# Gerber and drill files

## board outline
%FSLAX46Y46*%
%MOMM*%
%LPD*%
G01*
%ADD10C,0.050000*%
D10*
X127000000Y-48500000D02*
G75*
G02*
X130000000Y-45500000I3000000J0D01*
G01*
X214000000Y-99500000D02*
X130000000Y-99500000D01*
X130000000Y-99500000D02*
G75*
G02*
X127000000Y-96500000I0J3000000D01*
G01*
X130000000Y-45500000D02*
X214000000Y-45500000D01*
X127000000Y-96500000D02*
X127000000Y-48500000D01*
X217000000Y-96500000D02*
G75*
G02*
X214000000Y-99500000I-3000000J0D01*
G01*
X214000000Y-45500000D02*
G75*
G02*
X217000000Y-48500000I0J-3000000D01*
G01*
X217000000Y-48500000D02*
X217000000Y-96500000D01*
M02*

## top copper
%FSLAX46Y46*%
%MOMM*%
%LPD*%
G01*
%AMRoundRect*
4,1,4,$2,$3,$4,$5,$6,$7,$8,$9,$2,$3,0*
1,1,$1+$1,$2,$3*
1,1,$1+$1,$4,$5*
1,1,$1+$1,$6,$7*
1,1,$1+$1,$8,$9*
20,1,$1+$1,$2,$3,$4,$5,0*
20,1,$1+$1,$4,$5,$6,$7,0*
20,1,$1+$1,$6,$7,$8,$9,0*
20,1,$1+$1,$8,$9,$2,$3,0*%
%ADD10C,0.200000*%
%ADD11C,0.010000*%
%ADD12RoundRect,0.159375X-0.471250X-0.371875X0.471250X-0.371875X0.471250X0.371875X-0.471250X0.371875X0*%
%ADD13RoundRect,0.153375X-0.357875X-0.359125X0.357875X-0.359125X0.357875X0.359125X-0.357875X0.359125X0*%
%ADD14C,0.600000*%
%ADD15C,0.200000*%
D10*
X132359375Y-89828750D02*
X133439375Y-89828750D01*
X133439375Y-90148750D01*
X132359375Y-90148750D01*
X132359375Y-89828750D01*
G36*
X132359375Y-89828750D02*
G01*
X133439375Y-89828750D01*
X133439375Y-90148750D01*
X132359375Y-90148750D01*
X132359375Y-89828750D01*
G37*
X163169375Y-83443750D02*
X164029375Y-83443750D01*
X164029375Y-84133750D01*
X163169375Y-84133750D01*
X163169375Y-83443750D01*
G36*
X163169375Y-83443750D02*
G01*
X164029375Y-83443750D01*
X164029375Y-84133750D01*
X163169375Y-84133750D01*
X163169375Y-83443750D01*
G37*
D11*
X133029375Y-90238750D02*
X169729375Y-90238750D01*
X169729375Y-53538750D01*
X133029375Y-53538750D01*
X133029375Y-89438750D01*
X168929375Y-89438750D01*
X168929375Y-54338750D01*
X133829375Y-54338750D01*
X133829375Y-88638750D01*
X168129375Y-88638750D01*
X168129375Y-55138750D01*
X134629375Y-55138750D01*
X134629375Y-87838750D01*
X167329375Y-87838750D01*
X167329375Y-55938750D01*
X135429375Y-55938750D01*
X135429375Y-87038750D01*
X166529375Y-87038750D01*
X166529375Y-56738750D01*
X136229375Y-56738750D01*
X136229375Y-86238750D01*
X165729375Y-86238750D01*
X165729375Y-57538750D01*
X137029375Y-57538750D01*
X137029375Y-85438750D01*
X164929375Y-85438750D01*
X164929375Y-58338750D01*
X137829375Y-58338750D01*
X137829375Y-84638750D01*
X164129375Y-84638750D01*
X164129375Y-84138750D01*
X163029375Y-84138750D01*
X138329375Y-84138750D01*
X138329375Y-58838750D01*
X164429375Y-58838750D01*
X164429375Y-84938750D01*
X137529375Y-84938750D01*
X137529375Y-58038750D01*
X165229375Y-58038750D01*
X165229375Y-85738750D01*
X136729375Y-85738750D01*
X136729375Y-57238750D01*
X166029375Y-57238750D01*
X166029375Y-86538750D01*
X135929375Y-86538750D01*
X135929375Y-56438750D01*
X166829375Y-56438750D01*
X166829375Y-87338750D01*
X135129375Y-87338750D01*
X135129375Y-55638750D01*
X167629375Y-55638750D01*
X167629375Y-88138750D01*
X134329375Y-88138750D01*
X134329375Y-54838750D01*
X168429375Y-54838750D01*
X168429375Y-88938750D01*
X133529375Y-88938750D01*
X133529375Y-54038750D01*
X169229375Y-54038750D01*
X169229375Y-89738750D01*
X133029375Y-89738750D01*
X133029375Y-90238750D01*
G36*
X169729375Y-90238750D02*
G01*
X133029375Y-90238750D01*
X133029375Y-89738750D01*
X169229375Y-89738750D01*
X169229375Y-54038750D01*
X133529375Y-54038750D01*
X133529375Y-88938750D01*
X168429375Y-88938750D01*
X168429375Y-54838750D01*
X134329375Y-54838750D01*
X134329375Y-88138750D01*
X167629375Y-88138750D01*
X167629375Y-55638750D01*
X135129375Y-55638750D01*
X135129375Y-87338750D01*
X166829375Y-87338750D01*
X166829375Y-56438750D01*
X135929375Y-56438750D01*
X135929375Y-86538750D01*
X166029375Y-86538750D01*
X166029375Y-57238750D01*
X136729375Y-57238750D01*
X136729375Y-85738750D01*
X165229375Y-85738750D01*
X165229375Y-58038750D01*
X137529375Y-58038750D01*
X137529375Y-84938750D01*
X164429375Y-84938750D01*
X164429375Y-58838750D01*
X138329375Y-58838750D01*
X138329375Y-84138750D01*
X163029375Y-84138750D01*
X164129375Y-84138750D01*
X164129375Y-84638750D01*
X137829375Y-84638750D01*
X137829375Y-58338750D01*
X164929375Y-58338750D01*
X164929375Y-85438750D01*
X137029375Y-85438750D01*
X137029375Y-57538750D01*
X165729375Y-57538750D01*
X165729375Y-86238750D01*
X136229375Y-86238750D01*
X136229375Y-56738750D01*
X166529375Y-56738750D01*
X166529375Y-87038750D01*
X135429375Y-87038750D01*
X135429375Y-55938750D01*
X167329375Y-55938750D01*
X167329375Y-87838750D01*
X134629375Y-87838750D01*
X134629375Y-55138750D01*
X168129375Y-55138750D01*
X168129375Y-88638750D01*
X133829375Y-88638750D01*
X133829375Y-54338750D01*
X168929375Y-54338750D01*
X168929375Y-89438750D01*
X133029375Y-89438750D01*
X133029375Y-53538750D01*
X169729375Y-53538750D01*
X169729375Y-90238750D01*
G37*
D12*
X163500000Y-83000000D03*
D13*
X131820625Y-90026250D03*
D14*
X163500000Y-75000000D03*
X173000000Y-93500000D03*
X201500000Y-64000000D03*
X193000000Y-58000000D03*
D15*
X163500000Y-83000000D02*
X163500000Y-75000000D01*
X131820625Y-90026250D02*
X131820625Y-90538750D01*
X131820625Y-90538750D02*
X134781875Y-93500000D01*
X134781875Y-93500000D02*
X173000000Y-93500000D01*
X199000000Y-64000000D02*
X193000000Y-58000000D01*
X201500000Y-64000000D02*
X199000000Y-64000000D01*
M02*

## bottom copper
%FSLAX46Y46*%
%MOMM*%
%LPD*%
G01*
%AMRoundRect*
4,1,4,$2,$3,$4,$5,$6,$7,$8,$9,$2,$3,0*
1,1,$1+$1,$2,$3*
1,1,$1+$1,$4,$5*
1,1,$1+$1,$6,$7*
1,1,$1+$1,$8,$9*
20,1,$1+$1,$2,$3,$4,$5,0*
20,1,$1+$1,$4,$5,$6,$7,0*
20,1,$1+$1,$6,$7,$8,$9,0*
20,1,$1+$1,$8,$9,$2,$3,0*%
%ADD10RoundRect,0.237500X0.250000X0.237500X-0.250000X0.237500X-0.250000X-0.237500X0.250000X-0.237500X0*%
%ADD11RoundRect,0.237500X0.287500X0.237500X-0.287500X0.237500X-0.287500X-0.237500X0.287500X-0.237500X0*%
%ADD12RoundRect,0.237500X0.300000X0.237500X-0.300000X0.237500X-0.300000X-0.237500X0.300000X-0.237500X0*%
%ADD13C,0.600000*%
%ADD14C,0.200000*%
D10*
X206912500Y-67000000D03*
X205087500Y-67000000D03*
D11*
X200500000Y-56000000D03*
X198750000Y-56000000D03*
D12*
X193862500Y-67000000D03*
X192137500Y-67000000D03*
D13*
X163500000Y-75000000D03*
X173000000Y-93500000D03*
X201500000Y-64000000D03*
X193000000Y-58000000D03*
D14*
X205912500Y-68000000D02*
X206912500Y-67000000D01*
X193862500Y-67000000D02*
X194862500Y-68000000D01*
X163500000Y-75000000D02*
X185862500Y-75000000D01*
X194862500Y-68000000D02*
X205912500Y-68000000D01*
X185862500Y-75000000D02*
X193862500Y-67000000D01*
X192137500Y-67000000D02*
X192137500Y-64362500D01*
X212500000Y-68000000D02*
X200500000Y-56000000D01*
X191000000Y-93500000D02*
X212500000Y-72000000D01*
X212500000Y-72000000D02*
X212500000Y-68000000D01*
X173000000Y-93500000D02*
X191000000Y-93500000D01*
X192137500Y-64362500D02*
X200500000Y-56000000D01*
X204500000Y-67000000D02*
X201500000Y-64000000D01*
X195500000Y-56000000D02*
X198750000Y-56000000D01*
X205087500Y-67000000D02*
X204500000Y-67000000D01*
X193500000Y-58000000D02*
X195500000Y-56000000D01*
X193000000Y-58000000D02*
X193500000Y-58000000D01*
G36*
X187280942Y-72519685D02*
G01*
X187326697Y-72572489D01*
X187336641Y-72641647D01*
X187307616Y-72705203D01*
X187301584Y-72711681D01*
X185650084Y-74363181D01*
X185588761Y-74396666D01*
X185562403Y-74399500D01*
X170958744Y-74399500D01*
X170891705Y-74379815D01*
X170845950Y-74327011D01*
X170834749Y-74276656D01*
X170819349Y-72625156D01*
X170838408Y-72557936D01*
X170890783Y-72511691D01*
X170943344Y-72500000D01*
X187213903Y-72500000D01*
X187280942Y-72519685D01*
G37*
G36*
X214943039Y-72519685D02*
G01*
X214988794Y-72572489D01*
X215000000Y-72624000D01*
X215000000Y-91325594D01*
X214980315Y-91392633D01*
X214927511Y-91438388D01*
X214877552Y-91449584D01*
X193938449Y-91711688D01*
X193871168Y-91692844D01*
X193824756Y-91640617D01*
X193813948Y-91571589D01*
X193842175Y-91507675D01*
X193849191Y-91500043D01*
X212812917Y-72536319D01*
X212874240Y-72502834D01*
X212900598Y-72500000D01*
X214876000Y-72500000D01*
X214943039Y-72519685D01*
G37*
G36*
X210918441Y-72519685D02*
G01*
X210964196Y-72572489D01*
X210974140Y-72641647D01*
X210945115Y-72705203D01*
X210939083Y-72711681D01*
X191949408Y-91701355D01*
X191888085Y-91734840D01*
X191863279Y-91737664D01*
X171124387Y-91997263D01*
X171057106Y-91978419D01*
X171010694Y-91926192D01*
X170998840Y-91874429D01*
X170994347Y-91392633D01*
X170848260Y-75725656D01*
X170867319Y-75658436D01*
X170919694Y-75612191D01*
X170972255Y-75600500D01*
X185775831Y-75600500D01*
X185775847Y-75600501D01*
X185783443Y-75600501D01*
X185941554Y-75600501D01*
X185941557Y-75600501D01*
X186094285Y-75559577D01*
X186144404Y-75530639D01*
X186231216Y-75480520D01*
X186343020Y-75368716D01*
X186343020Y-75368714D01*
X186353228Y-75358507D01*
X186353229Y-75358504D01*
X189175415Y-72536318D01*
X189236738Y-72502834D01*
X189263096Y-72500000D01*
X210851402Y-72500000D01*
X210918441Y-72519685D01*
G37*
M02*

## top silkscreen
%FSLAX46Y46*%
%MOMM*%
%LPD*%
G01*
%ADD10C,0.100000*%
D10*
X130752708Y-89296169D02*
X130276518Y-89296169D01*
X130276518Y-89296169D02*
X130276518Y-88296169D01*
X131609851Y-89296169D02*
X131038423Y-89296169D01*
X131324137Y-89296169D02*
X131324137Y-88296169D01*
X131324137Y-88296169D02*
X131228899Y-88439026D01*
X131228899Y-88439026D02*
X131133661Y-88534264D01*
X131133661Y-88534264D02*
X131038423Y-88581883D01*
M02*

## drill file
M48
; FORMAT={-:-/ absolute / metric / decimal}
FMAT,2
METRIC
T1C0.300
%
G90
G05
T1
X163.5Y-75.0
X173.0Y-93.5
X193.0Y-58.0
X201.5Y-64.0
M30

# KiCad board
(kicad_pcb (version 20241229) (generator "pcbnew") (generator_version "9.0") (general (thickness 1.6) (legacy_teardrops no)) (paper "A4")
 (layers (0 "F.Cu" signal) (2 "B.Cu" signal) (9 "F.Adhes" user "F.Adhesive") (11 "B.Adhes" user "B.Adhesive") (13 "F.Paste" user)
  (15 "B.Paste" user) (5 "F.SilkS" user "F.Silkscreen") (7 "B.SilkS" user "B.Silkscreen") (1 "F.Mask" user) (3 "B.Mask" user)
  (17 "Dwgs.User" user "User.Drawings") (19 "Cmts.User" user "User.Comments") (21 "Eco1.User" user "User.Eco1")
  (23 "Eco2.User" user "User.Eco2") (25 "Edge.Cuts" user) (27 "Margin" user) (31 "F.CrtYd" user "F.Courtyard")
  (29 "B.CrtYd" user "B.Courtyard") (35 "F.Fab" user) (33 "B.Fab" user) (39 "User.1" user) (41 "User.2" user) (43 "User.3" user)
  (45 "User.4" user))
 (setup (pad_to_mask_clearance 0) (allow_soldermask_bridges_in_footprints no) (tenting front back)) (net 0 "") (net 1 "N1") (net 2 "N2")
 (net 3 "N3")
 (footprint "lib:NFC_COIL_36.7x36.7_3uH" (layer "F.Cu") (at 133.029375 90.23875)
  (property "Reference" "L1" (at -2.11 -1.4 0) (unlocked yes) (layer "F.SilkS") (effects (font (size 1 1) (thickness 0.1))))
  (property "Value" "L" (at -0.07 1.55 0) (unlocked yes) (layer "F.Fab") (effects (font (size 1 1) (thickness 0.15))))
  (fp_rect (start -0.67 -0.41) (end 0.41 -0.09) (stroke (width 0.2) (type solid)) (fill yes) (layer "F.Cu"))
  (fp_rect (start 30.14 -6.795) (end 31 -6.105) (stroke (width 0.2) (type solid)) (fill yes) (layer "F.Cu"))
  (fp_poly
   (pts (xy 0 0) (xy 36.7 0) (xy 36.7 -36.7) (xy 0 -36.7) (xy 0 -0.8) (xy 35.9 -0.8) (xy 35.9 -35.9) (xy 0.8 -35.9) (xy 0.8 -1.6)
    (xy 35.1 -1.6) (xy 35.1 -35.1) (xy 1.6 -35.1) (xy 1.6 -2.4) (xy 34.3 -2.4) (xy 34.3 -34.3) (xy 2.4 -34.3) (xy 2.4 -3.2) (xy 33.5 -3.2)
    (xy 33.5 -33.5) (xy 3.2 -33.5) (xy 3.2 -4) (xy 32.7 -4) (xy 32.7 -32.7) (xy 4 -32.7) (xy 4 -4.8) (xy 31.9 -4.8) (xy 31.9 -31.9)
    (xy 4.8 -31.9) (xy 4.8 -5.6) (xy 31.1 -5.6) (xy 31.1 -6.1) (xy 30 -6.1) (xy 5.3 -6.1) (xy 5.3 -31.4) (xy 31.4 -31.4) (xy 31.4 -5.3)
    (xy 4.5 -5.3) (xy 4.5 -32.2) (xy 32.2 -32.2) (xy 32.2 -4.5) (xy 3.7 -4.5) (xy 3.7 -33) (xy 33 -33) (xy 33 -3.7) (xy 2.9 -3.7)
    (xy 2.9 -33.8) (xy 33.8 -33.8) (xy 33.8 -2.9) (xy 2.1 -2.9) (xy 2.1 -34.6) (xy 34.6 -34.6) (xy 34.6 -2.1) (xy 1.3 -2.1) (xy 1.3 -35.4)
    (xy 35.4 -35.4) (xy 35.4 -1.3) (xy 0.5 -1.3) (xy 0.5 -36.2) (xy 36.2 -36.2) (xy 36.2 -0.5) (xy 0 -0.5))
   (stroke (width 0.01) (type solid)) (fill yes) (layer "F.Cu"))
  (pad "1" smd roundrect (at 30.470625 -7.23875) (size 1.26125 1.0625) (layers "F.Cu" "F.Mask" "F.Paste") (roundrect_rratio 0.15)
   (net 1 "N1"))
  (pad "2" smd roundrect (at -1.20875 -0.2125) (size 1.0225 1.025) (layers "F.Cu" "F.Mask" "F.Paste") (roundrect_rratio 0.15) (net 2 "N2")))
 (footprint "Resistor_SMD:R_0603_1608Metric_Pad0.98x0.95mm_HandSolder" (layer "B.Cu") (at 206 67 180)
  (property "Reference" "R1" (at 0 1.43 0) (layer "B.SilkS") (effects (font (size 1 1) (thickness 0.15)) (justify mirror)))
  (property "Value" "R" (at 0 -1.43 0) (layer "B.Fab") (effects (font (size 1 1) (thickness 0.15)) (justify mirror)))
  (pad "1" smd roundrect (at -0.9125 0 180) (size 0.975 0.95) (layers "B.Cu" "B.Mask" "B.Paste") (roundrect_rratio 0.25) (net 1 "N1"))
  (pad "2" smd roundrect (at 0.9125 0 180) (size 0.975 0.95) (layers "B.Cu" "B.Mask" "B.Paste") (roundrect_rratio 0.25) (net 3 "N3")))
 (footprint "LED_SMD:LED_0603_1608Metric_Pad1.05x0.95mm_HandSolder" (layer "B.Cu") (at 199.625 56 180)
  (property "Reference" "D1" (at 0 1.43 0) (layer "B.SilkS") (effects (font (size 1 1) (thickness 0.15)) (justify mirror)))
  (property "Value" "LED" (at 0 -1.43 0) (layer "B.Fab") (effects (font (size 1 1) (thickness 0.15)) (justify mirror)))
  (pad "1" smd roundrect (at -0.875 0 180) (size 1.05 0.95) (layers "B.Cu" "B.Mask" "B.Paste") (roundrect_rratio 0.25) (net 2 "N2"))
  (pad "2" smd roundrect (at 0.875 0 180) (size 1.05 0.95) (layers "B.Cu" "B.Mask" "B.Paste") (roundrect_rratio 0.25) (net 3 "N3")))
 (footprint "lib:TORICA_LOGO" (layer "B.Cu") (at 193 59.5 180)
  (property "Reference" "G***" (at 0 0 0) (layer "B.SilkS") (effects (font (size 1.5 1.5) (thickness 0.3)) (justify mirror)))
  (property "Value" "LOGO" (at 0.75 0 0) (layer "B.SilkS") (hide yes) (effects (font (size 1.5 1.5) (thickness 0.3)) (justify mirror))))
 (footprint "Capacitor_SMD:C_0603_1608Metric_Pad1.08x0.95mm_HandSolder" (layer "B.Cu") (at 193 67 180)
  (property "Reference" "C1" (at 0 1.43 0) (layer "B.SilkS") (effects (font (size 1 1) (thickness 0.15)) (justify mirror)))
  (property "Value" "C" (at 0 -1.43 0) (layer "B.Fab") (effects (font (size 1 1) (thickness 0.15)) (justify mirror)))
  (pad "1" smd roundrect (at -0.8625 0 180) (size 1.075 0.95) (layers "B.Cu" "B.Mask" "B.Paste") (roundrect_rratio 0.25) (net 1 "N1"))
  (pad "2" smd roundrect (at 0.8625 0 180) (size 1.075 0.95) (layers "B.Cu" "B.Mask" "B.Paste") (roundrect_rratio 0.25) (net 2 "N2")))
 (gr_arc (start 127 48.5) (mid 127.87868 46.37868) (end 130 45.5) (stroke (width 0.05) (type default)) (layer "Edge.Cuts"))
 (gr_line (start 214 99.5) (end 130 99.5) (stroke (width 0.05) (type default)) (layer "Edge.Cuts"))
 (gr_arc (start 130 99.5) (mid 127.87868 98.62132) (end 127 96.5) (stroke (width 0.05) (type default)) (layer "Edge.Cuts"))
 (gr_line (start 130 45.5) (end 214 45.5) (stroke (width 0.05) (type default)) (layer "Edge.Cuts"))
 (gr_line (start 127 96.5) (end 127 48.5) (stroke (width 0.05) (type default)) (layer "Edge.Cuts"))
 (gr_arc (start 217 96.5) (mid 216.12132 98.62132) (end 214 99.5) (stroke (width 0.05) (type default)) (layer "Edge.Cuts"))
 (gr_arc (start 214 45.5) (mid 216.12132 46.37868) (end 217 48.5) (stroke (width 0.05) (type default)) (layer "Edge.Cuts"))
 (gr_line (start 217 48.5) (end 217 96.5) (stroke (width 0.05) (type default)) (layer "Edge.Cuts"))
 (segment (start 163.5 83) (end 163.5 75) (width 0.2) (layer "F.Cu") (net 1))
 (via (at 163.5 75) (size 0.6) (drill 0.3) (layers "F.Cu" "B.Cu") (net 1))
 (segment (start 205.9125 68) (end 206.9125 67) (width 0.2) (layer "B.Cu") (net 1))
 (segment (start 193.8625 67) (end 194.8625 68) (width 0.2) (layer "B.Cu") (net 1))
 (segment (start 163.5 75) (end 185.8625 75) (width 0.2) (layer "B.Cu") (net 1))
 (segment (start 194.8625 68) (end 205.9125 68) (width 0.2) (layer "B.Cu") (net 1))
 (segment (start 185.8625 75) (end 193.8625 67) (width 0.2) (layer "B.Cu") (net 1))
 (segment (start 131.820625 90.02625) (end 131.820625 90.53875) (width 0.2) (layer "F.Cu") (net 2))
 (segment (start 131.820625 90.53875) (end 134.781875 93.5) (width 0.2) (layer "F.Cu") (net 2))
 (segment (start 134.781875 93.5) (end 173 93.5) (width 0.2) (layer "F.Cu") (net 2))
 (via (at 173 93.5) (size 0.6) (drill 0.3) (layers "F.Cu" "B.Cu") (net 2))
 (segment (start 192.1375 67) (end 192.1375 64.3625) (width 0.2) (layer "B.Cu") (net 2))
 (segment (start 212.5 68) (end 200.5 56) (width 0.2) (layer "B.Cu") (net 2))
 (segment (start 191 93.5) (end 212.5 72) (width 0.2) (layer "B.Cu") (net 2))
 (segment (start 212.5 72) (end 212.5 68) (width 0.2) (layer "B.Cu") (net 2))
 (segment (start 173 93.5) (end 191 93.5) (width 0.2) (layer "B.Cu") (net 2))
 (segment (start 192.1375 64.3625) (end 200.5 56) (width 0.2) (layer "B.Cu") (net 2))
 (segment (start 199 64) (end 193 58) (width 0.2) (layer "F.Cu") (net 3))
 (segment (start 201.5 64) (end 199 64) (width 0.2) (layer "F.Cu") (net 3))
 (via (at 201.5 64) (size 0.6) (drill 0.3) (layers "F.Cu" "B.Cu") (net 3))
 (via (at 193 58) (size 0.6) (drill 0.3) (layers "F.Cu" "B.Cu") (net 3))
 (segment (start 204.5 67) (end 201.5 64) (width 0.2) (layer "B.Cu") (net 3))
 (segment (start 195.5 56) (end 198.75 56) (width 0.2) (layer "B.Cu") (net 3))
 (segment (start 205.0875 67) (end 204.5 67) (width 0.2) (layer "B.Cu") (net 3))
 (segment (start 193.5 58) (end 195.5 56) (width 0.2) (layer "B.Cu") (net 3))
 (segment (start 193 58) (end 193.5 58) (width 0.2) (layer "B.Cu") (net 3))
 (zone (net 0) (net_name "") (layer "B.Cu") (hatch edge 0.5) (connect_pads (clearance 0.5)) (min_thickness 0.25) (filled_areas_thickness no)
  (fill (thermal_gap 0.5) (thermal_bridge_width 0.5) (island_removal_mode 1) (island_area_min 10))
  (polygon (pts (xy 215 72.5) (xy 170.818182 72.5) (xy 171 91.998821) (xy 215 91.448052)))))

